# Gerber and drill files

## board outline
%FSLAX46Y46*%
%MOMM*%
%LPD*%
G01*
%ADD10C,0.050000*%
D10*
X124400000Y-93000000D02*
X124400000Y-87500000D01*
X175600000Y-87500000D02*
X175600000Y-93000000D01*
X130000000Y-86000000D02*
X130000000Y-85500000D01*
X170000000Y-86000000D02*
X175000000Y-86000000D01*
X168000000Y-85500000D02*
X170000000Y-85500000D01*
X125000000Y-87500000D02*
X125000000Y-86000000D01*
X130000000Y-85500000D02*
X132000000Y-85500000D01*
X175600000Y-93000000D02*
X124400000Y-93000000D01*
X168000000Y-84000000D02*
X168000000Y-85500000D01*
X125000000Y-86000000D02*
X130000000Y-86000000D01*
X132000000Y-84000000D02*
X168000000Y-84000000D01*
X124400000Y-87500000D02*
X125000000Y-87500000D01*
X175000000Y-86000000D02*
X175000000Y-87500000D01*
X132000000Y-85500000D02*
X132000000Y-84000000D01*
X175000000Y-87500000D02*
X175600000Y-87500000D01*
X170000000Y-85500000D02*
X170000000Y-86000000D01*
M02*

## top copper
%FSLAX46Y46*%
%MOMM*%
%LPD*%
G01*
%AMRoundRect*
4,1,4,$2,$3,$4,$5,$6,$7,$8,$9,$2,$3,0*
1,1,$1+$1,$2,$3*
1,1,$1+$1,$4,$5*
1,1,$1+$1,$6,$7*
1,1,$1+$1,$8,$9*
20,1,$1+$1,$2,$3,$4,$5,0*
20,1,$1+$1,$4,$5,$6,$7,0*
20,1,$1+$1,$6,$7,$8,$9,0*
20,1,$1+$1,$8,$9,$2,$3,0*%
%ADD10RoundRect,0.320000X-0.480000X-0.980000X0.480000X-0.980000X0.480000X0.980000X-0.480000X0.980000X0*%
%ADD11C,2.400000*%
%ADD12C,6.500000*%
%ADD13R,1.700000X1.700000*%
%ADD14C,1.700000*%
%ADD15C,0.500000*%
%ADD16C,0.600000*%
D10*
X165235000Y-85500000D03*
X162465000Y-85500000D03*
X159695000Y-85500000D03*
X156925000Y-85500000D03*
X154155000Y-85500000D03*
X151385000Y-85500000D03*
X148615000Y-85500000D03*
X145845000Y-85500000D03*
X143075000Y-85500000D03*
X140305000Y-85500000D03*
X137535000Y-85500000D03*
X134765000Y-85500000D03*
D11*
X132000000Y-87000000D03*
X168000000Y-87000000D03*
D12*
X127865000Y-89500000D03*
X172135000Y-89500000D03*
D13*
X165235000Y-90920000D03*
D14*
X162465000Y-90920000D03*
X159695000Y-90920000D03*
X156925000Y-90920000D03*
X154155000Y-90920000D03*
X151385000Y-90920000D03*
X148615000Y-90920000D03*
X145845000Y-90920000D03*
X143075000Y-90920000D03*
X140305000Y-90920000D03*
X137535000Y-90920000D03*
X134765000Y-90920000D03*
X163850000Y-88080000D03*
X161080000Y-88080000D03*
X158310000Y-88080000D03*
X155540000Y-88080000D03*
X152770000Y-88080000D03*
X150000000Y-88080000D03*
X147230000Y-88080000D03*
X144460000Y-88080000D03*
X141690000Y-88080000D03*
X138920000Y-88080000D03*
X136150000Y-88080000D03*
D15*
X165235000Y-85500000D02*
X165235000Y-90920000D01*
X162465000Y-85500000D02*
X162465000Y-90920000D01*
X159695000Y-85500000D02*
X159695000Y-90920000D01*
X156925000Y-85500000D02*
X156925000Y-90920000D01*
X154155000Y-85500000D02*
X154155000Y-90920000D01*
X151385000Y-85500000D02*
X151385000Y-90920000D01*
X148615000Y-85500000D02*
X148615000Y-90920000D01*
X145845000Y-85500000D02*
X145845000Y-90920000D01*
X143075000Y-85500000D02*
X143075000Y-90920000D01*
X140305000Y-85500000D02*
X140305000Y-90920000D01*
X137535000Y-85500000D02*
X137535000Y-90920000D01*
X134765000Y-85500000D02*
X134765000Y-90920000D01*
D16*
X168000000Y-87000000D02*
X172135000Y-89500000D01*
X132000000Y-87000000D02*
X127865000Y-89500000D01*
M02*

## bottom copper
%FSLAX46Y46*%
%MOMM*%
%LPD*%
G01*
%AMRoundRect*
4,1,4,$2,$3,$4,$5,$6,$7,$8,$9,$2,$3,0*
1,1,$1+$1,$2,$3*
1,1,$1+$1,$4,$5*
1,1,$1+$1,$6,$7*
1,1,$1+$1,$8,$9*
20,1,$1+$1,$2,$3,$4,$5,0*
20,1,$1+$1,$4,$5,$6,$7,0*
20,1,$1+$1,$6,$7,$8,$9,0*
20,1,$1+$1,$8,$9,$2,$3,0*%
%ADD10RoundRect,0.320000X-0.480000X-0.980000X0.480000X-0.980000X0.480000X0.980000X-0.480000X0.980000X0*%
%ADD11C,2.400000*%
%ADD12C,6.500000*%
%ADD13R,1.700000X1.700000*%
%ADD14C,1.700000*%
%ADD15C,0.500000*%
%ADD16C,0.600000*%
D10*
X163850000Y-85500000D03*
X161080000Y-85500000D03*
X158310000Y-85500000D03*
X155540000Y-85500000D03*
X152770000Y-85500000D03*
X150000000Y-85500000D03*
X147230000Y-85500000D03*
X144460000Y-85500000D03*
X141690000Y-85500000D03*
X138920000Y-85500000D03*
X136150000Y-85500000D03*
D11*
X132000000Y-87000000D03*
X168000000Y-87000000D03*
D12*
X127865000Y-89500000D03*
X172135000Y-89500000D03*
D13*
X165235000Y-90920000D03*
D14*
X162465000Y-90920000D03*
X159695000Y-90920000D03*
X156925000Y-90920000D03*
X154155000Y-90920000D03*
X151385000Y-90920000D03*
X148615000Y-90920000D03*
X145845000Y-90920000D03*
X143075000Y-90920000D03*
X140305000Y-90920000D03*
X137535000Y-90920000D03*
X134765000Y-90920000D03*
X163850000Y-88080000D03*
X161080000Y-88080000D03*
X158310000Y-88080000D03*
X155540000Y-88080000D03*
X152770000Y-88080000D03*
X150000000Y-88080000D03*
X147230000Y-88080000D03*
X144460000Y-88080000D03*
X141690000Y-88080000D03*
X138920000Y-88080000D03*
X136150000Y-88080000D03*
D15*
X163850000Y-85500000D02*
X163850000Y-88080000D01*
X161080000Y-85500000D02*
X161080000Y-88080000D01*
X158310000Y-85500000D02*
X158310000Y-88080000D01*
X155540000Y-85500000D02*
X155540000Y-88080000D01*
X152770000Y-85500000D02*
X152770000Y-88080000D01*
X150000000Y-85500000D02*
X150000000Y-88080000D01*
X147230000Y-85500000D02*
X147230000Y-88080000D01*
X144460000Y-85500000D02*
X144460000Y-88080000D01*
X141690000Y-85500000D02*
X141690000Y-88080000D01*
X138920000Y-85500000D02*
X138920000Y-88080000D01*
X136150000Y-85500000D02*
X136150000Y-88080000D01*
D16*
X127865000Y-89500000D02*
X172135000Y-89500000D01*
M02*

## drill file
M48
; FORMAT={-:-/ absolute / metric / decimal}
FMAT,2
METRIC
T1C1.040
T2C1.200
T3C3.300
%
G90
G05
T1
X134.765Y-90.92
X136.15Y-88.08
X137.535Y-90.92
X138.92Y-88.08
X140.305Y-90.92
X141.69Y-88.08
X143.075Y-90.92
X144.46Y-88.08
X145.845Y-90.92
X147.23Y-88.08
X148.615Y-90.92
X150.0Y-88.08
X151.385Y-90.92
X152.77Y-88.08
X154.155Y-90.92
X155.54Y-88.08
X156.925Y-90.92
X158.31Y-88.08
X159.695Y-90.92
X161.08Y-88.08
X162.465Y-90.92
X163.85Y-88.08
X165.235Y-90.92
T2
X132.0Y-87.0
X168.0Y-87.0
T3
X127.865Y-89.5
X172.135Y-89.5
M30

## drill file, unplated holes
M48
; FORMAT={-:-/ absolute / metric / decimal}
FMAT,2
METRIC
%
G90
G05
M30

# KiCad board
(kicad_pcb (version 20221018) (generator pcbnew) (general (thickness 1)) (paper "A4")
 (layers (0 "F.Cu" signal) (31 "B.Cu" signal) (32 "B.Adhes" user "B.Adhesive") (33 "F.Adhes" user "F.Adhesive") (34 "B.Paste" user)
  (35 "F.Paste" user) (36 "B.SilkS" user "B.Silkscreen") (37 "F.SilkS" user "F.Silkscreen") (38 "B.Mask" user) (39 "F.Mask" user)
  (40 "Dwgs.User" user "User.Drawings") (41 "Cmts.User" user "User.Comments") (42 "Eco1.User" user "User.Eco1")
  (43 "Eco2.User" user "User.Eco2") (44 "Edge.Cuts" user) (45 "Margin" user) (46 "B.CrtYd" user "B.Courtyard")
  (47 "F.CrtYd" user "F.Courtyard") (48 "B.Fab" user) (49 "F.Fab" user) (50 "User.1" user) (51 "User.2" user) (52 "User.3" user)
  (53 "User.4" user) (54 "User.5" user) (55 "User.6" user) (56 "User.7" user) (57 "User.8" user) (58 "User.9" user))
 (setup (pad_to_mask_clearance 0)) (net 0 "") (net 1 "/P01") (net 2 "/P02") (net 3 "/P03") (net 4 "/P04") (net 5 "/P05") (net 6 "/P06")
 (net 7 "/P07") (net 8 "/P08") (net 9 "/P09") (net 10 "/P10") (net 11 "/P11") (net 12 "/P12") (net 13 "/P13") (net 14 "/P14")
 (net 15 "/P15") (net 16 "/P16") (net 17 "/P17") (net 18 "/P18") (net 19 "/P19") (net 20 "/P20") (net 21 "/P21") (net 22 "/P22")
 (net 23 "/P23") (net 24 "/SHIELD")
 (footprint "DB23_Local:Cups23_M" (layer "F.Cu") (at 150 80)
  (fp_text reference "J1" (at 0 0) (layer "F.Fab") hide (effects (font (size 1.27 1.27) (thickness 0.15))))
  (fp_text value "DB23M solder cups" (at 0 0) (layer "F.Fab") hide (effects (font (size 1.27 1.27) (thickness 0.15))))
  (pad "1" smd roundrect (at 15.235 5.5) (size 1.6 2.6) (layers "F.Cu" "F.Mask") (roundrect_rratio 0.2) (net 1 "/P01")
   (thermal_bridge_angle 45))
  (pad "2" smd roundrect (at 12.465 5.5) (size 1.6 2.6) (layers "F.Cu" "F.Mask") (roundrect_rratio 0.2) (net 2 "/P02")
   (thermal_bridge_angle 45))
  (pad "3" smd roundrect (at 9.695 5.5) (size 1.6 2.6) (layers "F.Cu" "F.Mask") (roundrect_rratio 0.2) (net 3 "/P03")
   (thermal_bridge_angle 45))
  (pad "4" smd roundrect (at 6.925 5.5) (size 1.6 2.6) (layers "F.Cu" "F.Mask") (roundrect_rratio 0.2) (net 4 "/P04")
   (thermal_bridge_angle 45))
  (pad "5" smd roundrect (at 4.155 5.5) (size 1.6 2.6) (layers "F.Cu" "F.Mask") (roundrect_rratio 0.2) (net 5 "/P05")
   (thermal_bridge_angle 45))
  (pad "6" smd roundrect (at 1.385 5.5) (size 1.6 2.6) (layers "F.Cu" "F.Mask") (roundrect_rratio 0.2) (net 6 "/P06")
   (thermal_bridge_angle 45))
  (pad "7" smd roundrect (at -1.385 5.5) (size 1.6 2.6) (layers "F.Cu" "F.Mask") (roundrect_rratio 0.2) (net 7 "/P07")
   (thermal_bridge_angle 45))
  (pad "8" smd roundrect (at -4.155 5.5) (size 1.6 2.6) (layers "F.Cu" "F.Mask") (roundrect_rratio 0.2) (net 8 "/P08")
   (thermal_bridge_angle 45))
  (pad "9" smd roundrect (at -6.925 5.5) (size 1.6 2.6) (layers "F.Cu" "F.Mask") (roundrect_rratio 0.2) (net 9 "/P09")
   (thermal_bridge_angle 45))
  (pad "10" smd roundrect (at -9.695 5.5) (size 1.6 2.6) (layers "F.Cu" "F.Mask") (roundrect_rratio 0.2) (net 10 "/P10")
   (thermal_bridge_angle 45))
  (pad "11" smd roundrect (at -12.465 5.5) (size 1.6 2.6) (layers "F.Cu" "F.Mask") (roundrect_rratio 0.2) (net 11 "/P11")
   (thermal_bridge_angle 45))
  (pad "12" smd roundrect (at -15.235 5.5) (size 1.6 2.6) (layers "F.Cu" "F.Mask") (roundrect_rratio 0.2) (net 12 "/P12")
   (thermal_bridge_angle 45))
  (pad "13" smd roundrect (at 13.85 5.5) (size 1.6 2.6) (layers "B.Cu" "B.Mask") (roundrect_rratio 0.2) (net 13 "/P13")
   (thermal_bridge_angle 45))
  (pad "14" smd roundrect (at 11.08 5.5) (size 1.6 2.6) (layers "B.Cu" "B.Mask") (roundrect_rratio 0.2) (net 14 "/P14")
   (thermal_bridge_angle 45))
  (pad "15" smd roundrect (at 8.31 5.5) (size 1.6 2.6) (layers "B.Cu" "B.Mask") (roundrect_rratio 0.2) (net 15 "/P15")
   (thermal_bridge_angle 45))
  (pad "16" smd roundrect (at 5.54 5.5) (size 1.6 2.6) (layers "B.Cu" "B.Mask") (roundrect_rratio 0.2) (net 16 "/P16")
   (thermal_bridge_angle 45))
  (pad "17" smd roundrect (at 2.77 5.5) (size 1.6 2.6) (layers "B.Cu" "B.Mask") (roundrect_rratio 0.2) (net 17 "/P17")
   (thermal_bridge_angle 45))
  (pad "18" smd roundrect (at 0 5.5) (size 1.6 2.6) (layers "B.Cu" "B.Mask") (roundrect_rratio 0.2) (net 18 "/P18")
   (thermal_bridge_angle 45))
  (pad "19" smd roundrect (at -2.77 5.5) (size 1.6 2.6) (layers "B.Cu" "B.Mask") (roundrect_rratio 0.2) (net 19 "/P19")
   (thermal_bridge_angle 45))
  (pad "20" smd roundrect (at -5.54 5.5) (size 1.6 2.6) (layers "B.Cu" "B.Mask") (roundrect_rratio 0.2) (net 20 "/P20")
   (thermal_bridge_angle 45))
  (pad "21" smd roundrect (at -8.31 5.5) (size 1.6 2.6) (layers "B.Cu" "B.Mask") (roundrect_rratio 0.2) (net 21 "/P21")
   (thermal_bridge_angle 45))
  (pad "22" smd roundrect (at -11.08 5.5) (size 1.6 2.6) (layers "B.Cu" "B.Mask") (roundrect_rratio 0.2) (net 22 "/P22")
   (thermal_bridge_angle 45))
  (pad "23" smd roundrect (at -13.85 5.5) (size 1.6 2.6) (layers "B.Cu" "B.Mask") (roundrect_rratio 0.2) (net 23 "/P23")
   (thermal_bridge_angle 45)))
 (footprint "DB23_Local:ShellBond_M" (layer "F.Cu") (at 150 80)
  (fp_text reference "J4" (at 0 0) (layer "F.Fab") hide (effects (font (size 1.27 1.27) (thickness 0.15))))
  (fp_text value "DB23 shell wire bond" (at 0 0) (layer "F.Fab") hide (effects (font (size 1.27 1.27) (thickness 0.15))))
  (pad "1" thru_hole circle (at -18 7) (size 2.4 2.4) (drill 1.2) (layers "*.Cu" "*.Mask") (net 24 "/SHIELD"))
  (pad "2" thru_hole circle (at 18 7) (size 2.4 2.4) (drill 1.2) (layers "*.Cu" "*.Mask") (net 24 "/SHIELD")))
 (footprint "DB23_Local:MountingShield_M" (layer "F.Cu") (at 150 80)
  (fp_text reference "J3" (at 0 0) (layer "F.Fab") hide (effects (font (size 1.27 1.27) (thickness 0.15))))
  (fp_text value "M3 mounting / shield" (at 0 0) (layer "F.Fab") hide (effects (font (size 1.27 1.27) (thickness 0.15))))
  (pad "1" thru_hole circle (at -22.135 9.5) (size 6.5 6.5) (drill 3.3) (layers "*.Cu" "*.Mask") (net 24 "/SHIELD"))
  (pad "2" thru_hole circle (at 22.135 9.5) (size 6.5 6.5) (drill 3.3) (layers "*.Cu" "*.Mask") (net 24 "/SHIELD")))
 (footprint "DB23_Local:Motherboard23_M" (layer "F.Cu") (at 150 80)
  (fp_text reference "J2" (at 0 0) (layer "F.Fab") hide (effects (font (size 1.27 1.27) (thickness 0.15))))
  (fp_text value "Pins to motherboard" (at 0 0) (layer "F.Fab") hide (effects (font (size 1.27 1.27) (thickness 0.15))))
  (pad "1" thru_hole rect (at 15.235 10.92) (size 1.7 1.7) (drill 1.04) (layers "*.Cu" "*.Mask") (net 1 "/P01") (thermal_bridge_angle 45))
  (pad "2" thru_hole circle (at 12.465 10.92) (size 1.7 1.7) (drill 1.04) (layers "*.Cu" "*.Mask") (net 2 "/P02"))
  (pad "3" thru_hole circle (at 9.695 10.92) (size 1.7 1.7) (drill 1.04) (layers "*.Cu" "*.Mask") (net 3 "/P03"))
  (pad "4" thru_hole circle (at 6.925 10.92) (size 1.7 1.7) (drill 1.04) (layers "*.Cu" "*.Mask") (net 4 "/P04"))
  (pad "5" thru_hole circle (at 4.155 10.92) (size 1.7 1.7) (drill 1.04) (layers "*.Cu" "*.Mask") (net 5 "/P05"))
  (pad "6" thru_hole circle (at 1.385 10.92) (size 1.7 1.7) (drill 1.04) (layers "*.Cu" "*.Mask") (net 6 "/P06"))
  (pad "7" thru_hole circle (at -1.385 10.92) (size 1.7 1.7) (drill 1.04) (layers "*.Cu" "*.Mask") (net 7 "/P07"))
  (pad "8" thru_hole circle (at -4.155 10.92) (size 1.7 1.7) (drill 1.04) (layers "*.Cu" "*.Mask") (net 8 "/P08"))
  (pad "9" thru_hole circle (at -6.925 10.92) (size 1.7 1.7) (drill 1.04) (layers "*.Cu" "*.Mask") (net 9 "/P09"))
  (pad "10" thru_hole circle (at -9.695 10.92) (size 1.7 1.7) (drill 1.04) (layers "*.Cu" "*.Mask") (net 10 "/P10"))
  (pad "11" thru_hole circle (at -12.465 10.92) (size 1.7 1.7) (drill 1.04) (layers "*.Cu" "*.Mask") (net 11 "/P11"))
  (pad "12" thru_hole circle (at -15.235 10.92) (size 1.7 1.7) (drill 1.04) (layers "*.Cu" "*.Mask") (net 12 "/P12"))
  (pad "13" thru_hole circle (at 13.85 8.08) (size 1.7 1.7) (drill 1.04) (layers "*.Cu" "*.Mask") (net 13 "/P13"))
  (pad "14" thru_hole circle (at 11.08 8.08) (size 1.7 1.7) (drill 1.04) (layers "*.Cu" "*.Mask") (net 14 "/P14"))
  (pad "15" thru_hole circle (at 8.31 8.08) (size 1.7 1.7) (drill 1.04) (layers "*.Cu" "*.Mask") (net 15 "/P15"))
  (pad "16" thru_hole circle (at 5.54 8.08) (size 1.7 1.7) (drill 1.04) (layers "*.Cu" "*.Mask") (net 16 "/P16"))
  (pad "17" thru_hole circle (at 2.77 8.08) (size 1.7 1.7) (drill 1.04) (layers "*.Cu" "*.Mask") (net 17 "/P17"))
  (pad "18" thru_hole circle (at 0 8.08) (size 1.7 1.7) (drill 1.04) (layers "*.Cu" "*.Mask") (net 18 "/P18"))
  (pad "19" thru_hole circle (at -2.77 8.08) (size 1.7 1.7) (drill 1.04) (layers "*.Cu" "*.Mask") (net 19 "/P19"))
  (pad "20" thru_hole circle (at -5.54 8.08) (size 1.7 1.7) (drill 1.04) (layers "*.Cu" "*.Mask") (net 20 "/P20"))
  (pad "21" thru_hole circle (at -8.31 8.08) (size 1.7 1.7) (drill 1.04) (layers "*.Cu" "*.Mask") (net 21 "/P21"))
  (pad "22" thru_hole circle (at -11.08 8.08) (size 1.7 1.7) (drill 1.04) (layers "*.Cu" "*.Mask") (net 22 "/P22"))
  (pad "23" thru_hole circle (at -13.85 8.08) (size 1.7 1.7) (drill 1.04) (layers "*.Cu" "*.Mask") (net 23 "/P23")))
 (gr_line (start 124.4 93) (end 124.4 87.5) (stroke (width 0.05) (type default)) (layer "Edge.Cuts"))
 (gr_line (start 175.6 87.5) (end 175.6 93) (stroke (width 0.05) (type default)) (layer "Edge.Cuts"))
 (gr_line (start 130 86) (end 130 85.5) (stroke (width 0.05) (type default)) (layer "Edge.Cuts"))
 (gr_line (start 170 86) (end 175 86) (stroke (width 0.05) (type default)) (layer "Edge.Cuts"))
 (gr_line (start 168 85.5) (end 170 85.5) (stroke (width 0.05) (type default)) (layer "Edge.Cuts"))
 (gr_line (start 125 87.5) (end 125 86) (stroke (width 0.05) (type default)) (layer "Edge.Cuts"))
 (gr_line (start 130 85.5) (end 132 85.5) (stroke (width 0.05) (type default)) (layer "Edge.Cuts"))
 (gr_line (start 175.6 93) (end 124.4 93) (stroke (width 0.05) (type default)) (layer "Edge.Cuts"))
 (gr_line (start 168 84) (end 168 85.5) (stroke (width 0.05) (type default)) (layer "Edge.Cuts"))
 (gr_line (start 125 86) (end 130 86) (stroke (width 0.05) (type default)) (layer "Edge.Cuts"))
 (gr_line (start 132 84) (end 168 84) (stroke (width 0.05) (type default)) (layer "Edge.Cuts"))
 (gr_line (start 124.4 87.5) (end 125 87.5) (stroke (width 0.05) (type default)) (layer "Edge.Cuts"))
 (gr_line (start 175 86) (end 175 87.5) (stroke (width 0.05) (type default)) (layer "Edge.Cuts"))
 (gr_line (start 132 85.5) (end 132 84) (stroke (width 0.05) (type default)) (layer "Edge.Cuts"))
 (gr_line (start 175 87.5) (end 175.6 87.5) (stroke (width 0.05) (type default)) (layer "Edge.Cuts"))
 (gr_line (start 170 85.5) (end 170 86) (stroke (width 0.05) (type default)) (layer "Edge.Cuts"))
 (segment (start 165.235 85.5) (end 165.235 90.92) (width 0.5) (layer "F.Cu") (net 1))
 (segment (start 162.465 85.5) (end 162.465 90.92) (width 0.5) (layer "F.Cu") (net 2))
 (segment (start 159.695 85.5) (end 159.695 90.92) (width 0.5) (layer "F.Cu") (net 3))
 (segment (start 156.925 85.5) (end 156.925 90.92) (width 0.5) (layer "F.Cu") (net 4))
 (segment (start 154.155 85.5) (end 154.155 90.92) (width 0.5) (layer "F.Cu") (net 5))
 (segment (start 151.385 85.5) (end 151.385 90.92) (width 0.5) (layer "F.Cu") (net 6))
 (segment (start 148.615 85.5) (end 148.615 90.92) (width 0.5) (layer "F.Cu") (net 7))
 (segment (start 145.845 85.5) (end 145.845 90.92) (width 0.5) (layer "F.Cu") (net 8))
 (segment (start 143.075 85.5) (end 143.075 90.92) (width 0.5) (layer "F.Cu") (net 9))
 (segment (start 140.305 85.5) (end 140.305 90.92) (width 0.5) (layer "F.Cu") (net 10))
 (segment (start 137.535 85.5) (end 137.535 90.92) (width 0.5) (layer "F.Cu") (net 11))
 (segment (start 134.765 85.5) (end 134.765 90.92) (width 0.5) (layer "F.Cu") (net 12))
 (segment (start 163.85 85.5) (end 163.85 88.08) (width 0.5) (layer "B.Cu") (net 13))
 (segment (start 161.08 85.5) (end 161.08 88.08) (width 0.5) (layer "B.Cu") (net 14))
 (segment (start 158.31 85.5) (end 158.31 88.08) (width 0.5) (layer "B.Cu") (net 15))
 (segment (start 155.54 85.5) (end 155.54 88.08) (width 0.5) (layer "B.Cu") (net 16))
 (segment (start 152.77 85.5) (end 152.77 88.08) (width 0.5) (layer "B.Cu") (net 17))
 (segment (start 150 85.5) (end 150 88.08) (width 0.5) (layer "B.Cu") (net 18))
 (segment (start 147.23 85.5) (end 147.23 88.08) (width 0.5) (layer "B.Cu") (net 19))
 (segment (start 144.46 85.5) (end 144.46 88.08) (width 0.5) (layer "B.Cu") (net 20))
 (segment (start 141.69 85.5) (end 141.69 88.08) (width 0.5) (layer "B.Cu") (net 21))
 (segment (start 138.92 85.5) (end 138.92 88.08) (width 0.5) (layer "B.Cu") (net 22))
 (segment (start 136.15 85.5) (end 136.15 88.08) (width 0.5) (layer "B.Cu") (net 23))
 (segment (start 168 87) (end 172.135 89.5) (width 0.6) (layer "F.Cu") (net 24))
 (segment (start 132 87) (end 127.865 89.5) (width 0.6) (layer "F.Cu") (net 24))
 (segment (start 127.865 89.5) (end 172.135 89.5) (width 0.6) (layer "B.Cu") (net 24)))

